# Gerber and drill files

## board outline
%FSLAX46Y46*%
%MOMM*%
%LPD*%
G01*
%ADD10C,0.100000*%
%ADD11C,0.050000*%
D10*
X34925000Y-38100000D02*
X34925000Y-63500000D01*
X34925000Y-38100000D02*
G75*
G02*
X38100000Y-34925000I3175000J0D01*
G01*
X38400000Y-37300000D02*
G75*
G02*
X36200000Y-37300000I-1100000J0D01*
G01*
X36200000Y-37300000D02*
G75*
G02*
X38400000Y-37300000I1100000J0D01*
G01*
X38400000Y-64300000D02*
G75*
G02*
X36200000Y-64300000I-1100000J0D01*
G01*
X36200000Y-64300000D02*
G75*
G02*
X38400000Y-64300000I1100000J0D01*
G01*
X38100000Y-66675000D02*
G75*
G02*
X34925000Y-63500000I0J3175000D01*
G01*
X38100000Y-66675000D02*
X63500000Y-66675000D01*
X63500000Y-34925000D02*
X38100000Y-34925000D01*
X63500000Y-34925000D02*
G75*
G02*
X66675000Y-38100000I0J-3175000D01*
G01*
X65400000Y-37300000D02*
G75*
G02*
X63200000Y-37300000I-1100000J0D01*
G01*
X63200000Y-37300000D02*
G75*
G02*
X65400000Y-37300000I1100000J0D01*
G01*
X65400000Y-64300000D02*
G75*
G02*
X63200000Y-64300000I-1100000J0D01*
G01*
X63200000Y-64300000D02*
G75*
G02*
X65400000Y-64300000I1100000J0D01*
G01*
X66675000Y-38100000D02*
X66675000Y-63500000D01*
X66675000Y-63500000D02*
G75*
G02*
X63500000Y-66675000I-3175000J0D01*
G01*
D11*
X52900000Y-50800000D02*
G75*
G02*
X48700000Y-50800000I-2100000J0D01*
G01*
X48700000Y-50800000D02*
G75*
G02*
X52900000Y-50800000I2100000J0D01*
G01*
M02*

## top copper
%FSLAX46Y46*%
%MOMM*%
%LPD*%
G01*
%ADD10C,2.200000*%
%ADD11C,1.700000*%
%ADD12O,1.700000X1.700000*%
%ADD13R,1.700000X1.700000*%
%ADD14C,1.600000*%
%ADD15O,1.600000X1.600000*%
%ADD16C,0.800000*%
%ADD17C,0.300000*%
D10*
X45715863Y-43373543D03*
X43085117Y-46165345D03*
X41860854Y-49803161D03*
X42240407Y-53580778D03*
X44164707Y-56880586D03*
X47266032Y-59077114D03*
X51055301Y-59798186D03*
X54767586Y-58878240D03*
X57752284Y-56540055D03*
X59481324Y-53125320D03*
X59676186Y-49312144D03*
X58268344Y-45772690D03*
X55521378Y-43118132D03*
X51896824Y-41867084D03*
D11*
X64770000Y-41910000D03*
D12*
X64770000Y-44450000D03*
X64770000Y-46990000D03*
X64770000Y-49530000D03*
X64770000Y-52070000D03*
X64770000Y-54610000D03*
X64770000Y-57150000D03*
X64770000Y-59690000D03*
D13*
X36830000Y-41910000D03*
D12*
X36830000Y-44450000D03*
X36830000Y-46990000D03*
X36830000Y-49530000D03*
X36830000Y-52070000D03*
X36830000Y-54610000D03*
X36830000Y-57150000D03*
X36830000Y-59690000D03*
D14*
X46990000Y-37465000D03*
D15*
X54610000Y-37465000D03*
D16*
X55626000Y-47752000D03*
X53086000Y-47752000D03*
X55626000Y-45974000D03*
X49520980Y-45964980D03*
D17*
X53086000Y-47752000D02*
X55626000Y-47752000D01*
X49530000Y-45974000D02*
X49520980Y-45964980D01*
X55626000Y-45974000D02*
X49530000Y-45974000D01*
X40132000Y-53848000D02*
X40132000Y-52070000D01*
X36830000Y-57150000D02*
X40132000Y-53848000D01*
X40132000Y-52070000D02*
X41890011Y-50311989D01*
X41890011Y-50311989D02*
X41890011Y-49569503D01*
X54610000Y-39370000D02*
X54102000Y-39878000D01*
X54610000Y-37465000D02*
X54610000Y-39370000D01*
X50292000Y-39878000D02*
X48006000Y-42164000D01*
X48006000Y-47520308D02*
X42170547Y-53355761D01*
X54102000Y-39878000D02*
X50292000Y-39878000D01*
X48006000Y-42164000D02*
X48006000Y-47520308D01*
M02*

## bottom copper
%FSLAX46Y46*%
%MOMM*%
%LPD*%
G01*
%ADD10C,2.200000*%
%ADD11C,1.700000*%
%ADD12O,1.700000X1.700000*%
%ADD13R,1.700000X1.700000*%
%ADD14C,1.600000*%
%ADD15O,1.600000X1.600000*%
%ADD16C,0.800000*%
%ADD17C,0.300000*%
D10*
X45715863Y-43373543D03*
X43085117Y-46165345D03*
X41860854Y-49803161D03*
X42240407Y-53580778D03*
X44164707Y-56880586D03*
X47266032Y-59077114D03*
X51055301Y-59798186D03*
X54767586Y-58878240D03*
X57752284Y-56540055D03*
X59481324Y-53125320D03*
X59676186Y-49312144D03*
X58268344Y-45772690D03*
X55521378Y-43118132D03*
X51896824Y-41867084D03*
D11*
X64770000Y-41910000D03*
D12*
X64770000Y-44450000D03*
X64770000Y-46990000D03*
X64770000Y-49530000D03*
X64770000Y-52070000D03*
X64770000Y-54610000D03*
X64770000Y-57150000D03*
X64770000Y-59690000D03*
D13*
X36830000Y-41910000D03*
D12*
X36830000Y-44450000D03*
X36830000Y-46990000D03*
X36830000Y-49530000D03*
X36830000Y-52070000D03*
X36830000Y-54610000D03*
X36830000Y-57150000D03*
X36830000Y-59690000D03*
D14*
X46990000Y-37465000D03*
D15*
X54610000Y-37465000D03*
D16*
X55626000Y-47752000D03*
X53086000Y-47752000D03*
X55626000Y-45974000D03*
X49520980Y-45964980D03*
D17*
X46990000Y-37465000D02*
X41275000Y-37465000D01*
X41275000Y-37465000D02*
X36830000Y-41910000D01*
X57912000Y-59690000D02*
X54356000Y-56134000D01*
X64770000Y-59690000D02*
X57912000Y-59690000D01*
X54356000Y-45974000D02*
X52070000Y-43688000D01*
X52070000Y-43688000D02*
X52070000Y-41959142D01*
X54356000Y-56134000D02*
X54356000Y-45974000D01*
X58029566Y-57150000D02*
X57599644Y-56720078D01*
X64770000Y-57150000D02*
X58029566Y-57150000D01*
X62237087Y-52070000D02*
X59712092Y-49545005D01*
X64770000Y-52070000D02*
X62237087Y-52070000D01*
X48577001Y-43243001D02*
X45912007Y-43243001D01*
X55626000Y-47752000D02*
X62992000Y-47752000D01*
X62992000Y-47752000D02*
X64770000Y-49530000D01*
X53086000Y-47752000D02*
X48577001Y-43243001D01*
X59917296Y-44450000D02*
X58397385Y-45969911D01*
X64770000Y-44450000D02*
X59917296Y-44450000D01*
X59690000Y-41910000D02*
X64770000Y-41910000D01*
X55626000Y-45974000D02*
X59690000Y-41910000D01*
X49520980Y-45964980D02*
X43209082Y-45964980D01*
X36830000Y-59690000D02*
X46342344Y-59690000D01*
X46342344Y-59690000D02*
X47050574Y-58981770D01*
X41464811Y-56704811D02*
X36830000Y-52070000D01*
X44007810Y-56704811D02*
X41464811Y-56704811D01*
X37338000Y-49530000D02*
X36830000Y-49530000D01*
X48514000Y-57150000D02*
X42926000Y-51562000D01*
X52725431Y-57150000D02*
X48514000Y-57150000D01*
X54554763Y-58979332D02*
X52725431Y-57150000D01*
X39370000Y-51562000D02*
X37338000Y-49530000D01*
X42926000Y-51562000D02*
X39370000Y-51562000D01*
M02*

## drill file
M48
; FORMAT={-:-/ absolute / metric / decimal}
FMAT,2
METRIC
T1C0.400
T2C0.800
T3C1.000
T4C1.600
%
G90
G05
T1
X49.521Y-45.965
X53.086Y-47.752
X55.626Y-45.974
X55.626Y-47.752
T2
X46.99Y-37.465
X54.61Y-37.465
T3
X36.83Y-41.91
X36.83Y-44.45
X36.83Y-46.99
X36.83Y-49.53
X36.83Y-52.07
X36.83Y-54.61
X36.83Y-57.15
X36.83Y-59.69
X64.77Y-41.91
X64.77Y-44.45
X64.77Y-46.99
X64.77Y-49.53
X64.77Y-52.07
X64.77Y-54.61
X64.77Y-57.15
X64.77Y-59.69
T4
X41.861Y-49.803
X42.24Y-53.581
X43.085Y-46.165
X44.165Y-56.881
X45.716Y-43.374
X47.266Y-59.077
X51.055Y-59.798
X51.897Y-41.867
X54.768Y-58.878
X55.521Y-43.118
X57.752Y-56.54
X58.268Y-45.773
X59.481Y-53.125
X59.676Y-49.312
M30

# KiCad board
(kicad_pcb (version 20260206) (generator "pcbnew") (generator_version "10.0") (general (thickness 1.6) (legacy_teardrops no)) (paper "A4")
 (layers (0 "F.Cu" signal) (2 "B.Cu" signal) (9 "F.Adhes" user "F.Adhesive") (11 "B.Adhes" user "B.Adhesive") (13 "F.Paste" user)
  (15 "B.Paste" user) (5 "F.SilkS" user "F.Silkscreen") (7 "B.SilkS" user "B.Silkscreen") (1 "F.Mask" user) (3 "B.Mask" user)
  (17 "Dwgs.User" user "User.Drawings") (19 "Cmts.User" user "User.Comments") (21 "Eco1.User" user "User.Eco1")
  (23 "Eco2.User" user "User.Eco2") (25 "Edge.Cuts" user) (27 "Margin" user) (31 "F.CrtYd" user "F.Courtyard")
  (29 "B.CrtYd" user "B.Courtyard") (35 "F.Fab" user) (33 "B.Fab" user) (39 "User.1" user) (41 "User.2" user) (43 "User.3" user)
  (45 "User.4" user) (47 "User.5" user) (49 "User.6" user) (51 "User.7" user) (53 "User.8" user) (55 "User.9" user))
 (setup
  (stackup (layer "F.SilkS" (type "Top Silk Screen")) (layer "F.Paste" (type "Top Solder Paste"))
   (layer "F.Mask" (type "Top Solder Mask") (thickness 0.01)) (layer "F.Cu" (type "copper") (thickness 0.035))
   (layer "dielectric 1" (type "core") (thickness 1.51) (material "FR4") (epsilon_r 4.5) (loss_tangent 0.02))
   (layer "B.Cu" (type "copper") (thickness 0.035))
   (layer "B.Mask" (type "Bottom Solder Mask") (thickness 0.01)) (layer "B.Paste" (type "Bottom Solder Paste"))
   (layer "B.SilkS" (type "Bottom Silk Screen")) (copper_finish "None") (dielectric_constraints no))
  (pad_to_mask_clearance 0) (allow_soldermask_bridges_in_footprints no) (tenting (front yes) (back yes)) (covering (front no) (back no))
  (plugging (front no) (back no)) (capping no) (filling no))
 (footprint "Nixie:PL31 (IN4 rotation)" (layer "F.Cu") (at 50.8 50.8 180)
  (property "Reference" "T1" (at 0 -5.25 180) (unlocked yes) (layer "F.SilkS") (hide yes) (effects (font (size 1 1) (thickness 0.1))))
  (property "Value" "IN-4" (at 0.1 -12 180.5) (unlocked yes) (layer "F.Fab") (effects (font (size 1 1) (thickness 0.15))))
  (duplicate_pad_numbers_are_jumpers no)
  (fp_circle (center 0 0) (end 2.09928 -0.054972) (stroke (width 0.05) (type default)) (fill no) (layer "Edge.Cuts"))
  (pad "1" thru_hole circle (at 5.084137 7.426457 353) (size 2.2 2.2) (drill 1.6) (layers "*.Cu" "*.Mask") (remove_unused_layers no)
   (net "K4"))
  (pad "2" thru_hole circle (at 7.714883 4.634655 353) (size 2.2 2.2) (drill 1.6) (layers "*.Cu" "*.Mask") (remove_unused_layers no)
   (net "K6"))
  (pad "3" thru_hole circle (at 8.939146 0.996839 353) (size 2.2 2.2) (drill 1.6) (layers "*.Cu" "*.Mask") (remove_unused_layers no)
   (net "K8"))
  (pad "4" thru_hole circle (at 8.559593 -2.780778 353) (size 2.2 2.2) (drill 1.6) (layers "*.Cu" "*.Mask") (remove_unused_layers no)
   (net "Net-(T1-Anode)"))
  (pad "5" thru_hole circle (at 6.635293 -6.080586 353) (size 2.2 2.2) (drill 1.6) (layers "*.Cu" "*.Mask") (remove_unused_layers no)
   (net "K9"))
  (pad "6" thru_hole circle (at 3.533968 -8.277114 353) (size 2.2 2.2) (drill 1.6) (layers "*.Cu" "*.Mask") (remove_unused_layers no)
   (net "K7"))
  (pad "7" thru_hole circle (at -0.255301 -8.998186 353) (size 2.2 2.2) (drill 1.6) (layers "*.Cu" "*.Mask") (remove_unused_layers no)
   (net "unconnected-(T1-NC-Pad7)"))
  (pad "8" thru_hole circle (at -3.967586 -8.07824 353) (size 2.2 2.2) (drill 1.6) (layers "*.Cu" "*.Mask") (remove_unused_layers no)
   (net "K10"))
  (pad "9" thru_hole circle (at -6.952284 -5.740055 353) (size 2.2 2.2) (drill 1.6) (layers "*.Cu" "*.Mask") (remove_unused_layers no)
   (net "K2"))
  (pad "10" thru_hole circle (at -8.681324 -2.32532 353) (size 2.2 2.2) (drill 1.6) (layers "*.Cu" "*.Mask") (remove_unused_layers no)
   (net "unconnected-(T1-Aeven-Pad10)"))
  (pad "11" thru_hole circle (at -8.876186 1.487856 353) (size 2.2 2.2) (drill 1.6) (layers "*.Cu" "*.Mask") (remove_unused_layers no)
   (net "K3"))
  (pad "12" thru_hole circle (at -7.468344 5.02731 353) (size 2.2 2.2) (drill 1.6) (layers "*.Cu" "*.Mask") (remove_unused_layers no)
   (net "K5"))
  (pad "13" thru_hole circle (at -4.721378 7.681868 353) (size 2.2 2.2) (drill 1.6) (layers "*.Cu" "*.Mask") (remove_unused_layers no)
   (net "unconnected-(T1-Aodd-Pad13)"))
  (pad "14" thru_hole circle (at -1.096824 8.932916 353) (size 2.2 2.2) (drill 1.6) (layers "*.Cu" "*.Mask") (remove_unused_layers no)
   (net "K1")))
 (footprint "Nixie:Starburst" (layer "F.Cu") (at 43 63.25)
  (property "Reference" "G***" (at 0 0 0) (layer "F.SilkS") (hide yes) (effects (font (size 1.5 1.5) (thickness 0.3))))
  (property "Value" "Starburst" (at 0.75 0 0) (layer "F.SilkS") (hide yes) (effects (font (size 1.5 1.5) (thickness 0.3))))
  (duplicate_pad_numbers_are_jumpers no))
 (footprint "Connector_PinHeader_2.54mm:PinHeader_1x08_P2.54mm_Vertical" (layer "B.Cu") (at 64.77 41.91 180)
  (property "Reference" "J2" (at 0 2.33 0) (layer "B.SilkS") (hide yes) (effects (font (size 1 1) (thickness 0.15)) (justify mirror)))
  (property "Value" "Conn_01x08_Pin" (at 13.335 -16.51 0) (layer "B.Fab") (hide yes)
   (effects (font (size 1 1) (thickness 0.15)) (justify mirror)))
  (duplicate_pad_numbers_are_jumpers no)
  (pad "1" thru_hole circle (at 0 0 180) (size 1.7 1.7) (drill 1) (layers "*.Cu" "*.Mask") (remove_unused_layers no) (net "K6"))
  (pad "2" thru_hole oval (at 0 -2.54 180) (size 1.7 1.7) (drill 1) (layers "*.Cu" "*.Mask") (remove_unused_layers no) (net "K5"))
  (pad "3" thru_hole oval (at 0 -5.08 180) (size 1.7 1.7) (drill 1) (layers "*.Cu" "*.Mask") (remove_unused_layers no)
   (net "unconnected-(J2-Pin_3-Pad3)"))
  (pad "4" thru_hole oval (at 0 -7.62 180) (size 1.7 1.7) (drill 1) (layers "*.Cu" "*.Mask") (remove_unused_layers no) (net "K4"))
  (pad "5" thru_hole oval (at 0 -10.16 180) (size 1.7 1.7) (drill 1) (layers "*.Cu" "*.Mask") (remove_unused_layers no) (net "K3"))
  (pad "6" thru_hole oval (at 0 -12.7 180) (size 1.7 1.7) (drill 1) (layers "*.Cu" "*.Mask") (remove_unused_layers no)
   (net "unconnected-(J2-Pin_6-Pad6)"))
  (pad "7" thru_hole oval (at 0 -15.24 180) (size 1.7 1.7) (drill 1) (layers "*.Cu" "*.Mask") (remove_unused_layers no) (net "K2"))
  (pad "8" thru_hole oval (at 0 -17.78 180) (size 1.7 1.7) (drill 1) (layers "*.Cu" "*.Mask") (remove_unused_layers no) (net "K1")))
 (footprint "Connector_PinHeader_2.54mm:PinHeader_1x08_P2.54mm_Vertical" (layer "B.Cu") (at 36.83 41.91 180)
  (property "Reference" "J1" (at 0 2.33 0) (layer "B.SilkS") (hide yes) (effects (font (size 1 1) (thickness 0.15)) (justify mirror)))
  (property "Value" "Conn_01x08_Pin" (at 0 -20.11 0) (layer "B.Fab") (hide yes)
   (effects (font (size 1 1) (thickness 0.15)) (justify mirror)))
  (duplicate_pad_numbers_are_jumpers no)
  (pad "1" thru_hole rect (at 0 0 180) (size 1.7 1.7) (drill 1) (layers "*.Cu" "*.Mask") (remove_unused_layers no) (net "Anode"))
  (pad "2" thru_hole oval (at 0 -2.54 180) (size 1.7 1.7) (drill 1) (layers "*.Cu" "*.Mask") (remove_unused_layers no)
   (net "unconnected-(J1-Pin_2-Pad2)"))
  (pad "3" thru_hole oval (at 0 -5.08 180) (size 1.7 1.7) (drill 1) (layers "*.Cu" "*.Mask") (remove_unused_layers no)
   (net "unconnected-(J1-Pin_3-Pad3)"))
  (pad "4" thru_hole oval (at 0 -7.62 180) (size 1.7 1.7) (drill 1) (layers "*.Cu" "*.Mask") (remove_unused_layers no) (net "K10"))
  (pad "5" thru_hole oval (at 0 -10.16 180) (size 1.7 1.7) (drill 1) (layers "*.Cu" "*.Mask") (remove_unused_layers no) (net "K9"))
  (pad "6" thru_hole oval (at 0 -12.7 180) (size 1.7 1.7) (drill 1) (layers "*.Cu" "*.Mask") (remove_unused_layers no)
   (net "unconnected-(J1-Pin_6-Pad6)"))
  (pad "7" thru_hole oval (at 0 -15.24 180) (size 1.7 1.7) (drill 1) (layers "*.Cu" "*.Mask") (remove_unused_layers no) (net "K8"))
  (pad "8" thru_hole oval (at 0 -17.78 180) (size 1.7 1.7) (drill 1) (layers "*.Cu" "*.Mask") (remove_unused_layers no) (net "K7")))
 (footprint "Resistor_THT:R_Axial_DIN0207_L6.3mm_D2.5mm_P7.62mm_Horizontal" (layer "B.Cu") (at 46.99 37.465)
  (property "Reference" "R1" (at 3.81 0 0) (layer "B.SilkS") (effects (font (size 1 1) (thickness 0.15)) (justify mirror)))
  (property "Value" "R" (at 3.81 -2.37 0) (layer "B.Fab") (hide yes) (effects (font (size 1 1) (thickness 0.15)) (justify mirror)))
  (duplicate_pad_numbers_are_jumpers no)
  (pad "1" thru_hole circle (at 0 0) (size 1.6 1.6) (drill 0.8) (layers "*.Cu" "*.Mask") (remove_unused_layers no) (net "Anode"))
  (pad "2" thru_hole oval (at 7.62 0) (size 1.6 1.6) (drill 0.8) (layers "*.Cu" "*.Mask") (remove_unused_layers no) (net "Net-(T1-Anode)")))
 (gr_line (start 34.925 38.1) (end 34.925 63.5) (stroke (width 0.1) (type default)) (layer "Edge.Cuts"))
 (gr_arc (start 34.925 38.1) (mid 35.854936 35.854936) (end 38.1 34.925) (stroke (width 0.1) (type default)) (layer "Edge.Cuts"))
 (gr_circle (center 37.3 37.3) (end 38.4 37.3) (stroke (width 0.1) (type default)) (fill no) (layer "Edge.Cuts"))
 (gr_circle (center 37.3 64.3) (end 38.4 64.3) (stroke (width 0.1) (type default)) (fill no) (layer "Edge.Cuts"))
 (gr_arc (start 38.1 66.675) (mid 35.854936 65.745064) (end 34.925 63.5) (stroke (width 0.1) (type default)) (layer "Edge.Cuts"))
 (gr_line (start 38.1 66.675) (end 63.5 66.675) (stroke (width 0.1) (type default)) (layer "Edge.Cuts"))
 (gr_line (start 63.5 34.925) (end 38.1 34.925) (stroke (width 0.1) (type default)) (layer "Edge.Cuts"))
 (gr_arc (start 63.5 34.925) (mid 65.745064 35.854936) (end 66.675 38.1) (stroke (width 0.1) (type default)) (layer "Edge.Cuts"))
 (gr_circle (center 64.3 37.3) (end 65.4 37.3) (stroke (width 0.1) (type default)) (fill no) (layer "Edge.Cuts"))
 (gr_circle (center 64.3 64.3) (end 65.4 64.3) (stroke (width 0.1) (type default)) (fill no) (layer "Edge.Cuts"))
 (gr_line (start 66.675 38.1) (end 66.675 63.5) (stroke (width 0.1) (type default)) (layer "Edge.Cuts"))
 (gr_arc (start 66.675 63.5) (mid 65.745064 65.745064) (end 63.5 66.675) (stroke (width 0.1) (type default)) (layer "Edge.Cuts"))
 (segment (start 46.99 37.465) (end 41.275 37.465) (width 0.3) (layer "B.Cu") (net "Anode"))
 (segment (start 41.275 37.465) (end 36.83 41.91) (width 0.3) (layer "B.Cu") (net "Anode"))
 (segment (start 57.912 59.69) (end 54.356 56.134) (width 0.3) (layer "B.Cu") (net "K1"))
 (segment (start 64.77 59.69) (end 57.912 59.69) (width 0.3) (layer "B.Cu") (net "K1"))
 (segment (start 54.356 45.974) (end 52.07 43.688) (width 0.3) (layer "B.Cu") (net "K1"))
 (segment (start 52.07 43.688) (end 52.07 41.959142) (width 0.3) (layer "B.Cu") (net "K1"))
 (segment (start 54.356 56.134) (end 54.356 45.974) (width 0.3) (layer "B.Cu") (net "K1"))
 (segment (start 58.029566 57.15) (end 57.599644 56.720078) (width 0.3) (layer "B.Cu") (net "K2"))
 (segment (start 64.77 57.15) (end 58.029566 57.15) (width 0.3) (layer "B.Cu") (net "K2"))
 (segment (start 62.237087 52.07) (end 59.712092 49.545005) (width 0.3) (layer "B.Cu") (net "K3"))
 (segment (start 64.77 52.07) (end 62.237087 52.07) (width 0.3) (layer "B.Cu") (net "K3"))
 (segment (start 53.086 47.752) (end 55.626 47.752) (width 0.3) (layer "F.Cu") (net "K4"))
 (via (at 55.626 47.752) (size 0.8) (drill 0.4) (layers "F.Cu" "B.Cu") (capping no) (covering (front no) (back no))
  (plugging (front no) (back no)) (filling no) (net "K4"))
 (via (at 53.086 47.752) (size 0.8) (drill 0.4) (layers "F.Cu" "B.Cu") (capping no) (covering (front no) (back no))
  (plugging (front no) (back no)) (filling no) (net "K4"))
 (segment (start 48.577001 43.243001) (end 45.912007 43.243001) (width 0.3) (layer "B.Cu") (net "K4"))
 (segment (start 55.626 47.752) (end 62.992 47.752) (width 0.3) (layer "B.Cu") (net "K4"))
 (segment (start 62.992 47.752) (end 64.77 49.53) (width 0.3) (layer "B.Cu") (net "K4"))
 (segment (start 53.086 47.752) (end 48.577001 43.243001) (width 0.3) (layer "B.Cu") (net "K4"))
 (segment (start 59.917296 44.45) (end 58.397385 45.969911) (width 0.3) (layer "B.Cu") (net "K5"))
 (segment (start 64.77 44.45) (end 59.917296 44.45) (width 0.3) (layer "B.Cu") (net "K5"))
 (segment (start 49.53 45.974) (end 49.52098 45.96498) (width 0.3) (layer "F.Cu") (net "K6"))
 (segment (start 55.626 45.974) (end 49.53 45.974) (width 0.3) (layer "F.Cu") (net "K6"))
 (via (at 55.626 45.974) (size 0.8) (drill 0.4) (layers "F.Cu" "B.Cu") (capping no) (covering (front no) (back no))
  (plugging (front no) (back no)) (filling no) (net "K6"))
 (via (at 49.52098 45.96498) (size 0.8) (drill 0.4) (layers "F.Cu" "B.Cu") (capping no) (covering (front no) (back no))
  (plugging (front no) (back no)) (filling no) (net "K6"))
 (segment (start 59.69 41.91) (end 64.77 41.91) (width 0.3) (layer "B.Cu") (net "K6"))
 (segment (start 55.626 45.974) (end 59.69 41.91) (width 0.3) (layer "B.Cu") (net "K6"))
 (segment (start 49.52098 45.96498) (end 43.209082 45.96498) (width 0.3) (layer "B.Cu") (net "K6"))
 (segment (start 36.83 59.69) (end 46.342344 59.69) (width 0.3) (layer "B.Cu") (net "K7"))
 (segment (start 46.342344 59.69) (end 47.050574 58.98177) (width 0.3) (layer "B.Cu") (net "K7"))
 (segment (start 40.132 53.848) (end 40.132 52.07) (width 0.3) (layer "F.Cu") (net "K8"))
 (segment (start 36.83 57.15) (end 40.132 53.848) (width 0.3) (layer "F.Cu") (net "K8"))
 (segment (start 40.132 52.07) (end 41.890011 50.311989) (width 0.3) (layer "F.Cu") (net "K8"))
 (segment (start 41.890011 50.311989) (end 41.890011 49.569503) (width 0.3) (layer "F.Cu") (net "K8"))
 (segment (start 41.464811 56.704811) (end 36.83 52.07) (width 0.3) (layer "B.Cu") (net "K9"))
 (segment (start 44.00781 56.704811) (end 41.464811 56.704811) (width 0.3) (layer "B.Cu") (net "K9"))
 (segment (start 37.338 49.53) (end 36.83 49.53) (width 0.3) (layer "B.Cu") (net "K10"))
 (segment (start 48.514 57.15) (end 42.926 51.562) (width 0.3) (layer "B.Cu") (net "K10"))
 (segment (start 52.725431 57.15) (end 48.514 57.15) (width 0.3) (layer "B.Cu") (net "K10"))
 (segment (start 54.554763 58.979332) (end 52.725431 57.15) (width 0.3) (layer "B.Cu") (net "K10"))
 (segment (start 39.37 51.562) (end 37.338 49.53) (width 0.3) (layer "B.Cu") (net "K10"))
 (segment (start 42.926 51.562) (end 39.37 51.562) (width 0.3) (layer "B.Cu") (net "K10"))
 (segment (start 54.61 39.37) (end 54.102 39.878) (width 0.3) (layer "F.Cu") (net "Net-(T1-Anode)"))
 (segment (start 54.61 37.465) (end 54.61 39.37) (width 0.3) (layer "F.Cu") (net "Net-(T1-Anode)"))
 (segment (start 50.292 39.878) (end 48.006 42.164) (width 0.3) (layer "F.Cu") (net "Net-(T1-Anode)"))
 (segment (start 48.006 47.520308) (end 42.170547 53.355761) (width 0.3) (layer "F.Cu") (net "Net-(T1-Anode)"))
 (segment (start 54.102 39.878) (end 50.292 39.878) (width 0.3) (layer "F.Cu") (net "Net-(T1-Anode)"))
 (segment (start 48.006 42.164) (end 48.006 47.520308) (width 0.3) (layer "F.Cu") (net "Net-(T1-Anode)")))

